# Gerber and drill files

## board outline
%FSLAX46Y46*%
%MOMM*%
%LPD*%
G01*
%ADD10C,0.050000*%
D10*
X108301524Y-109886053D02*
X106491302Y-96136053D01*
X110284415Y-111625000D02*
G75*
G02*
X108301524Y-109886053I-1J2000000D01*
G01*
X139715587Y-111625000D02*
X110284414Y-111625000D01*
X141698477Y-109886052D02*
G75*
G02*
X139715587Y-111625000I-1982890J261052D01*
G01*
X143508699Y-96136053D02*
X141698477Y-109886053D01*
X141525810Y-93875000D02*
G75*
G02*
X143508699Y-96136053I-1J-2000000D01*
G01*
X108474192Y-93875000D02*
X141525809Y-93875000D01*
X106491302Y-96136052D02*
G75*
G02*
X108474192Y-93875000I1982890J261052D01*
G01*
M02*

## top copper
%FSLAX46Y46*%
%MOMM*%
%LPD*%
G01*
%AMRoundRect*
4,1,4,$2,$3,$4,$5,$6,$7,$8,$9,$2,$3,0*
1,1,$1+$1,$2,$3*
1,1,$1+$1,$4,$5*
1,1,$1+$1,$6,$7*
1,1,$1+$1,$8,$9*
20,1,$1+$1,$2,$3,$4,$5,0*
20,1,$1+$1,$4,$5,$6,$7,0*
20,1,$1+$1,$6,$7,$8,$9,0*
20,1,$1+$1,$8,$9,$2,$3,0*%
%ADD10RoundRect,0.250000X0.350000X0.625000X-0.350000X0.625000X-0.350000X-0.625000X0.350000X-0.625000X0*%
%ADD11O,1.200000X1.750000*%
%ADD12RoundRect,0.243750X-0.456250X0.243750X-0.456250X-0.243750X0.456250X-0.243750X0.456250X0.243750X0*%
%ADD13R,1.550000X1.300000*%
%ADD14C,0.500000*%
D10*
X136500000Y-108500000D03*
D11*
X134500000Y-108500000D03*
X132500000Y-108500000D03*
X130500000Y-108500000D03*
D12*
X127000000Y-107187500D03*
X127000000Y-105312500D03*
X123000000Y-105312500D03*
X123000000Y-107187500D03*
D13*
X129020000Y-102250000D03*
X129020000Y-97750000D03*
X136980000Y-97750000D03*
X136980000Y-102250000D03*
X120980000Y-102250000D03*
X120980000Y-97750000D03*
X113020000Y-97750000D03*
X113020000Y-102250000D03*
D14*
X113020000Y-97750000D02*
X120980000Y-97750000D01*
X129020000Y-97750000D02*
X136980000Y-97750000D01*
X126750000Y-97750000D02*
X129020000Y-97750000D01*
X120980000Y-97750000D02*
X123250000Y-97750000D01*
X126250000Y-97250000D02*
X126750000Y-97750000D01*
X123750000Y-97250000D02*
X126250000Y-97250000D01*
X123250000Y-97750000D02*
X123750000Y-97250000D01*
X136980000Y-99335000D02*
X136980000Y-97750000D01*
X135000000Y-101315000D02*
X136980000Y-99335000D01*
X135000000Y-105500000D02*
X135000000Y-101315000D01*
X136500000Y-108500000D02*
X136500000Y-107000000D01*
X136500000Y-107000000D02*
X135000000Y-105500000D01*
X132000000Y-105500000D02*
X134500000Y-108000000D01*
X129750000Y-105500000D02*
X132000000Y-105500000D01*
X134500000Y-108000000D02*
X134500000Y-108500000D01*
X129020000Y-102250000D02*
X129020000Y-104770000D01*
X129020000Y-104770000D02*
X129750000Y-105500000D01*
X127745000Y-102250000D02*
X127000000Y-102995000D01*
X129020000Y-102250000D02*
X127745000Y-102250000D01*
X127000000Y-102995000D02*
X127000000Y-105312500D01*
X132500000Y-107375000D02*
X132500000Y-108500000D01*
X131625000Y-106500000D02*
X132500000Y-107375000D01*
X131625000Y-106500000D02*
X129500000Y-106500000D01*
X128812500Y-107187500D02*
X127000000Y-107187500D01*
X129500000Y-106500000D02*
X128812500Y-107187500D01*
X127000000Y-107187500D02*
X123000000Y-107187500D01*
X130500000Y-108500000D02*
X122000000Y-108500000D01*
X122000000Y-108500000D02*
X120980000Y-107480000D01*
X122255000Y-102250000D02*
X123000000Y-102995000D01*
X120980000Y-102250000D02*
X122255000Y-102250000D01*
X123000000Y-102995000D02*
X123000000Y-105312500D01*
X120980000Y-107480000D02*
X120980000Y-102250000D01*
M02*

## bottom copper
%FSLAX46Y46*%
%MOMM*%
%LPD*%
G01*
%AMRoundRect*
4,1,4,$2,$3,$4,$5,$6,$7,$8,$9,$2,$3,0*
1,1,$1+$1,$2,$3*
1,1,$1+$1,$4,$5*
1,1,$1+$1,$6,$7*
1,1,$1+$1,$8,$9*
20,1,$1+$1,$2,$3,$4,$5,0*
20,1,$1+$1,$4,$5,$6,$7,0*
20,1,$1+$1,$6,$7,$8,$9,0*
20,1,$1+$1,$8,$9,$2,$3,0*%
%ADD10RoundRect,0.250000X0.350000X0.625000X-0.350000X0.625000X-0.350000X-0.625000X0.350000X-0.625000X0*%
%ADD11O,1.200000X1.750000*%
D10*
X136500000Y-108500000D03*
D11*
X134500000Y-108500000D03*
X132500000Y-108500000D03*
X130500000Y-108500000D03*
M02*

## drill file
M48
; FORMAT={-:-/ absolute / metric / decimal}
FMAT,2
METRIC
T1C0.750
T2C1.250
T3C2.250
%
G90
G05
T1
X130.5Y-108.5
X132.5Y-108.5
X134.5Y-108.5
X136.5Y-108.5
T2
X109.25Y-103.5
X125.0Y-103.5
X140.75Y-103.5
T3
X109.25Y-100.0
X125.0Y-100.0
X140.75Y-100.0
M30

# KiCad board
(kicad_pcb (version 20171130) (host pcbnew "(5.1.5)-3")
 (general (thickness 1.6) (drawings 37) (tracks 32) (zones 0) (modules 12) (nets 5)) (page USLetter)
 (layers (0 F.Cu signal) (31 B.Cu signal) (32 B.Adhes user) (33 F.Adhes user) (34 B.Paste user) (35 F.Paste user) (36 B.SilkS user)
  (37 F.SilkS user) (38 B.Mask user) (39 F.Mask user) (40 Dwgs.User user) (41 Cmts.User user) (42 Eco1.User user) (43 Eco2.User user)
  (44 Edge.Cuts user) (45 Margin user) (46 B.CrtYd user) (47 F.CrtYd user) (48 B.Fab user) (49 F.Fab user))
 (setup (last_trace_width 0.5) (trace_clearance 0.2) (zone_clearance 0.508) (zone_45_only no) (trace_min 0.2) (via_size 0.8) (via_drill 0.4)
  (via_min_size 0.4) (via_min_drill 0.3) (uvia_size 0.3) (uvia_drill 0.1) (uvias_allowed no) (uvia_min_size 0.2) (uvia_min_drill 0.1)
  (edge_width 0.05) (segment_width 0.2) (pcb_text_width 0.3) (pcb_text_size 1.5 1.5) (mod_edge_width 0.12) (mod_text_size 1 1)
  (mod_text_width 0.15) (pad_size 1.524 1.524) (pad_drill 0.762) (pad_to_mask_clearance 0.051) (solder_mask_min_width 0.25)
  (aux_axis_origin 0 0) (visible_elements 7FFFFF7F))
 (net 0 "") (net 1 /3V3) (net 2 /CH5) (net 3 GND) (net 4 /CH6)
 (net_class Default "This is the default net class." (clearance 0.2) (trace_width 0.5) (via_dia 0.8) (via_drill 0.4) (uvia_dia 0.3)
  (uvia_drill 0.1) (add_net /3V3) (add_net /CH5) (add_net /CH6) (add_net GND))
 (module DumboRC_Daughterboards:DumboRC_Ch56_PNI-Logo (layer B.Cu) (at 125 96.5 180)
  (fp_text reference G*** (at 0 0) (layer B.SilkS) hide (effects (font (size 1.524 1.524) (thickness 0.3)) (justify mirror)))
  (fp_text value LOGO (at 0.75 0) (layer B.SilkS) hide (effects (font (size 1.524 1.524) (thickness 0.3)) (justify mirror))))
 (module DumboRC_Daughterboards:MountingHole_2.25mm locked (layer F.Cu) (at 109.25 100)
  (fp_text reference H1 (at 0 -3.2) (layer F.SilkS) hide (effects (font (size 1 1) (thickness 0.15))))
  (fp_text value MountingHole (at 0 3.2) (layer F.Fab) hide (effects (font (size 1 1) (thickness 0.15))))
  (pad "" np_thru_hole circle (at 0 0 90) (size 2.25 2.25) (drill 2.25) (layers *.Cu *.Mask)))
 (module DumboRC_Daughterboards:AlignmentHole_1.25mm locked (layer F.Cu) (at 109.25 103.5)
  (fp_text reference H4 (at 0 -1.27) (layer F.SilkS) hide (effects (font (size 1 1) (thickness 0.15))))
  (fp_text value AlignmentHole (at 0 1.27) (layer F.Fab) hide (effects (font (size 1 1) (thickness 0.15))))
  (pad "" np_thru_hole circle (at 0 0 90) (size 1.25 1.25) (drill 1.25) (layers *.Cu *.Mask)))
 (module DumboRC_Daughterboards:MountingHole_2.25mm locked (layer F.Cu) (at 125 100)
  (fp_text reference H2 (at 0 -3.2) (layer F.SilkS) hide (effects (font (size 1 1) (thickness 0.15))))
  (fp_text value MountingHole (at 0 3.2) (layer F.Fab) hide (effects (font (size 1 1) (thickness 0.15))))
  (pad "" np_thru_hole circle (at 0 0 90) (size 2.25 2.25) (drill 2.25) (layers *.Cu *.Mask)))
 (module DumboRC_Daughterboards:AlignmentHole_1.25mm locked (layer F.Cu) (at 125 103.5)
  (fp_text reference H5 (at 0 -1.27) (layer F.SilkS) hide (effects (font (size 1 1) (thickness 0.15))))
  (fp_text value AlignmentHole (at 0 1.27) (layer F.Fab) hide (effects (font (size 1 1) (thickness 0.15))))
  (pad "" np_thru_hole circle (at 0 0 90) (size 1.25 1.25) (drill 1.25) (layers *.Cu *.Mask)))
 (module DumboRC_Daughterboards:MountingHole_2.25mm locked (layer F.Cu) (at 140.75 100)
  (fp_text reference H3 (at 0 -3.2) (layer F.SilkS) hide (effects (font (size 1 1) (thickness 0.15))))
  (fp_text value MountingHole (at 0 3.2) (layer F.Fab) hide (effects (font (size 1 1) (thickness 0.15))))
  (pad "" np_thru_hole circle (at 0 0 90) (size 2.25 2.25) (drill 2.25) (layers *.Cu *.Mask)))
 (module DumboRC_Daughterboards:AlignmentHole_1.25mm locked (layer F.Cu) (at 140.75 103.5)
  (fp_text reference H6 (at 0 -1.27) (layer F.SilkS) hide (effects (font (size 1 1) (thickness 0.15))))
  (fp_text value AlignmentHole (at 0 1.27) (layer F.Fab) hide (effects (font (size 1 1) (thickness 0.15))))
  (pad "" np_thru_hole circle (at 0 0 90) (size 1.25 1.25) (drill 1.25) (layers *.Cu *.Mask)))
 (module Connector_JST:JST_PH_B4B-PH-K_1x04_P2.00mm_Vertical (layer B.Cu) (at 136.5 108.5 180)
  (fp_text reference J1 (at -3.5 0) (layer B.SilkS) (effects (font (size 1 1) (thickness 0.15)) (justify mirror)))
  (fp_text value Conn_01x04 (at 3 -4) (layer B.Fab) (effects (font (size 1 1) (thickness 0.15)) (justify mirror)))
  (pad 1 thru_hole roundrect (at 0 0 180) (size 1.2 1.75) (drill 0.75) (layers *.Cu *.Mask) (roundrect_rratio 0.208333) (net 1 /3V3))
  (pad 2 thru_hole oval (at 2 0 180) (size 1.2 1.75) (drill 0.75) (layers *.Cu *.Mask) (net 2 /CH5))
  (pad 3 thru_hole oval (at 4 0 180) (size 1.2 1.75) (drill 0.75) (layers *.Cu *.Mask) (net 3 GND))
  (pad 4 thru_hole oval (at 6 0 180) (size 1.2 1.75) (drill 0.75) (layers *.Cu *.Mask) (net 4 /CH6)))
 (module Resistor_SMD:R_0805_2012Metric (layer F.Cu) (at 127 106.25 270)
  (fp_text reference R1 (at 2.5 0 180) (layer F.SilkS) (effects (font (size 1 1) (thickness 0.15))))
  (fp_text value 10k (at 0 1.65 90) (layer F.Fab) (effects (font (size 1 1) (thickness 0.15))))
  (pad 2 smd roundrect (at 0.9375 0 270) (size 0.975 1.4) (layers F.Cu F.Paste F.Mask) (roundrect_rratio 0.25) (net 3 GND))
  (pad 1 smd roundrect (at -0.9375 0 270) (size 0.975 1.4) (layers F.Cu F.Paste F.Mask) (roundrect_rratio 0.25) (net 2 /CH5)))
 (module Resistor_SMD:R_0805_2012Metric (layer F.Cu) (at 123 106.25 270)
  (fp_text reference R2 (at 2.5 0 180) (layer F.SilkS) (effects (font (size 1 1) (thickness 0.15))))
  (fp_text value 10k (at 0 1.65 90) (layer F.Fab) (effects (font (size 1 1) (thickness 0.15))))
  (pad 1 smd roundrect (at -0.9375 0 270) (size 0.975 1.4) (layers F.Cu F.Paste F.Mask) (roundrect_rratio 0.25) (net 4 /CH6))
  (pad 2 smd roundrect (at 0.9375 0 270) (size 0.975 1.4) (layers F.Cu F.Paste F.Mask) (roundrect_rratio 0.25) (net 3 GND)))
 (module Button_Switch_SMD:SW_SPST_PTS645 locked (layer F.Cu) (at 133 100)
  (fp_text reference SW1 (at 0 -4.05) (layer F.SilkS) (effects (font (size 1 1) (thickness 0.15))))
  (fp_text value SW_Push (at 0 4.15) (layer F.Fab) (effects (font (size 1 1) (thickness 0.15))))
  (pad 2 smd rect (at -3.98 2.25) (size 1.55 1.3) (layers F.Cu F.Paste F.Mask) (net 2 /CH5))
  (pad 1 smd rect (at -3.98 -2.25) (size 1.55 1.3) (layers F.Cu F.Paste F.Mask) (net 1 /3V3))
  (pad 1 smd rect (at 3.98 -2.25) (size 1.55 1.3) (layers F.Cu F.Paste F.Mask) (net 1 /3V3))
  (pad 2 smd rect (at 3.98 2.25) (size 1.55 1.3) (layers F.Cu F.Paste F.Mask) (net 2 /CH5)))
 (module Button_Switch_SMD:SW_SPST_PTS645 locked (layer F.Cu) (at 117 100)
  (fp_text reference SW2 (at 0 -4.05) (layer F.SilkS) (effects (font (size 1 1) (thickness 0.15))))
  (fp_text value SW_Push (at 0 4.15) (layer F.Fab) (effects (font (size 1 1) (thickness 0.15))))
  (pad 2 smd rect (at 3.98 2.25) (size 1.55 1.3) (layers F.Cu F.Paste F.Mask) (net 4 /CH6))
  (pad 1 smd rect (at 3.98 -2.25) (size 1.55 1.3) (layers F.Cu F.Paste F.Mask) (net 1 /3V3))
  (pad 1 smd rect (at -3.98 -2.25) (size 1.55 1.3) (layers F.Cu F.Paste F.Mask) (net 1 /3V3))
  (pad 2 smd rect (at -3.98 2.25) (size 1.55 1.3) (layers F.Cu F.Paste F.Mask) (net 4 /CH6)))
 (gr_line (start 108.301524 109.886053) (end 106.491302 96.136053) (layer Edge.Cuts) (width 0.05))
 (gr_arc (start 110.284414 109.625) (end 108.301524 109.886053) (angle -82.5) (layer Edge.Cuts) (width 0.05))
 (gr_line (start 139.715587 111.625) (end 110.284414 111.625) (layer Edge.Cuts) (width 0.05))
 (gr_arc (start 139.715587 109.625) (end 139.715587 111.625) (angle -82.5) (layer Edge.Cuts) (width 0.05))
 (gr_line (start 143.508699 96.136053) (end 141.698477 109.886053) (layer Edge.Cuts) (width 0.05))
 (gr_arc (start 141.525809 95.875) (end 143.508699 96.136053) (angle -97.5) (layer Edge.Cuts) (width 0.05))
 (gr_line (start 108.474192 93.875) (end 141.525809 93.875) (layer Edge.Cuts) (width 0.05))
 (gr_arc (start 108.474192 95.875) (end 108.474192 93.875) (angle -97.5) (layer Edge.Cuts) (width 0.05))
 (segment (start 113.02 97.75) (end 120.98 97.75) (width 0.5) (layer F.Cu) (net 1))
 (segment (start 129.02 97.75) (end 136.98 97.75) (width 0.5) (layer F.Cu) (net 1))
 (segment (start 126.75 97.75) (end 129.02 97.75) (width 0.5) (layer F.Cu) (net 1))
 (segment (start 120.98 97.75) (end 123.25 97.75) (width 0.5) (layer F.Cu) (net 1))
 (segment (start 126.25 97.25) (end 126.75 97.75) (width 0.5) (layer F.Cu) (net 1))
 (segment (start 123.75 97.25) (end 126.25 97.25) (width 0.5) (layer F.Cu) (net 1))
 (segment (start 123.25 97.75) (end 123.75 97.25) (width 0.5) (layer F.Cu) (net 1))
 (segment (start 136.98 99.335) (end 136.98 97.75) (width 0.5) (layer F.Cu) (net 1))
 (segment (start 135 101.315) (end 136.98 99.335) (width 0.5) (layer F.Cu) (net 1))
 (segment (start 135 105.5) (end 135 101.315) (width 0.5) (layer F.Cu) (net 1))
 (segment (start 136.5 108.5) (end 136.5 107) (width 0.5) (layer F.Cu) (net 1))
 (segment (start 136.5 107) (end 135 105.5) (width 0.5) (layer F.Cu) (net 1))
 (segment (start 132 105.5) (end 134.5 108) (width 0.5) (layer F.Cu) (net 2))
 (segment (start 129.75 105.5) (end 132 105.5) (width 0.5) (layer F.Cu) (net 2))
 (segment (start 134.5 108) (end 134.5 108.5) (width 0.5) (layer F.Cu) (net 2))
 (segment (start 129.02 102.25) (end 129.02 104.77) (width 0.5) (layer F.Cu) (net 2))
 (segment (start 129.02 104.77) (end 129.75 105.5) (width 0.5) (layer F.Cu) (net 2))
 (segment (start 127.745 102.25) (end 127 102.995) (width 0.5) (layer F.Cu) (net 2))
 (segment (start 129.02 102.25) (end 127.745 102.25) (width 0.5) (layer F.Cu) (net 2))
 (segment (start 127 102.995) (end 127 105.3125) (width 0.5) (layer F.Cu) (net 2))
 (segment (start 132.5 107.375) (end 132.5 108.5) (width 0.5) (layer F.Cu) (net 3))
 (segment (start 131.625 106.5) (end 132.5 107.375) (width 0.5) (layer F.Cu) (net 3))
 (segment (start 131.625 106.5) (end 129.5 106.5) (width 0.5) (layer F.Cu) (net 3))
 (segment (start 128.8125 107.1875) (end 127 107.1875) (width 0.5) (layer F.Cu) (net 3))
 (segment (start 129.5 106.5) (end 128.8125 107.1875) (width 0.5) (layer F.Cu) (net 3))
 (segment (start 127 107.1875) (end 123 107.1875) (width 0.5) (layer F.Cu) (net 3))
 (segment (start 130.5 108.5) (end 122 108.5) (width 0.5) (layer F.Cu) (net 4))
 (segment (start 122 108.5) (end 120.98 107.48) (width 0.5) (layer F.Cu) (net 4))
 (segment (start 122.255 102.25) (end 123 102.995) (width 0.5) (layer F.Cu) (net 4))
 (segment (start 120.98 102.25) (end 122.255 102.25) (width 0.5) (layer F.Cu) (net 4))
 (segment (start 123 102.995) (end 123 105.3125) (width 0.5) (layer F.Cu) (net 4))
 (segment (start 120.98 107.48) (end 120.98 102.25) (width 0.5) (layer F.Cu) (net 4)))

